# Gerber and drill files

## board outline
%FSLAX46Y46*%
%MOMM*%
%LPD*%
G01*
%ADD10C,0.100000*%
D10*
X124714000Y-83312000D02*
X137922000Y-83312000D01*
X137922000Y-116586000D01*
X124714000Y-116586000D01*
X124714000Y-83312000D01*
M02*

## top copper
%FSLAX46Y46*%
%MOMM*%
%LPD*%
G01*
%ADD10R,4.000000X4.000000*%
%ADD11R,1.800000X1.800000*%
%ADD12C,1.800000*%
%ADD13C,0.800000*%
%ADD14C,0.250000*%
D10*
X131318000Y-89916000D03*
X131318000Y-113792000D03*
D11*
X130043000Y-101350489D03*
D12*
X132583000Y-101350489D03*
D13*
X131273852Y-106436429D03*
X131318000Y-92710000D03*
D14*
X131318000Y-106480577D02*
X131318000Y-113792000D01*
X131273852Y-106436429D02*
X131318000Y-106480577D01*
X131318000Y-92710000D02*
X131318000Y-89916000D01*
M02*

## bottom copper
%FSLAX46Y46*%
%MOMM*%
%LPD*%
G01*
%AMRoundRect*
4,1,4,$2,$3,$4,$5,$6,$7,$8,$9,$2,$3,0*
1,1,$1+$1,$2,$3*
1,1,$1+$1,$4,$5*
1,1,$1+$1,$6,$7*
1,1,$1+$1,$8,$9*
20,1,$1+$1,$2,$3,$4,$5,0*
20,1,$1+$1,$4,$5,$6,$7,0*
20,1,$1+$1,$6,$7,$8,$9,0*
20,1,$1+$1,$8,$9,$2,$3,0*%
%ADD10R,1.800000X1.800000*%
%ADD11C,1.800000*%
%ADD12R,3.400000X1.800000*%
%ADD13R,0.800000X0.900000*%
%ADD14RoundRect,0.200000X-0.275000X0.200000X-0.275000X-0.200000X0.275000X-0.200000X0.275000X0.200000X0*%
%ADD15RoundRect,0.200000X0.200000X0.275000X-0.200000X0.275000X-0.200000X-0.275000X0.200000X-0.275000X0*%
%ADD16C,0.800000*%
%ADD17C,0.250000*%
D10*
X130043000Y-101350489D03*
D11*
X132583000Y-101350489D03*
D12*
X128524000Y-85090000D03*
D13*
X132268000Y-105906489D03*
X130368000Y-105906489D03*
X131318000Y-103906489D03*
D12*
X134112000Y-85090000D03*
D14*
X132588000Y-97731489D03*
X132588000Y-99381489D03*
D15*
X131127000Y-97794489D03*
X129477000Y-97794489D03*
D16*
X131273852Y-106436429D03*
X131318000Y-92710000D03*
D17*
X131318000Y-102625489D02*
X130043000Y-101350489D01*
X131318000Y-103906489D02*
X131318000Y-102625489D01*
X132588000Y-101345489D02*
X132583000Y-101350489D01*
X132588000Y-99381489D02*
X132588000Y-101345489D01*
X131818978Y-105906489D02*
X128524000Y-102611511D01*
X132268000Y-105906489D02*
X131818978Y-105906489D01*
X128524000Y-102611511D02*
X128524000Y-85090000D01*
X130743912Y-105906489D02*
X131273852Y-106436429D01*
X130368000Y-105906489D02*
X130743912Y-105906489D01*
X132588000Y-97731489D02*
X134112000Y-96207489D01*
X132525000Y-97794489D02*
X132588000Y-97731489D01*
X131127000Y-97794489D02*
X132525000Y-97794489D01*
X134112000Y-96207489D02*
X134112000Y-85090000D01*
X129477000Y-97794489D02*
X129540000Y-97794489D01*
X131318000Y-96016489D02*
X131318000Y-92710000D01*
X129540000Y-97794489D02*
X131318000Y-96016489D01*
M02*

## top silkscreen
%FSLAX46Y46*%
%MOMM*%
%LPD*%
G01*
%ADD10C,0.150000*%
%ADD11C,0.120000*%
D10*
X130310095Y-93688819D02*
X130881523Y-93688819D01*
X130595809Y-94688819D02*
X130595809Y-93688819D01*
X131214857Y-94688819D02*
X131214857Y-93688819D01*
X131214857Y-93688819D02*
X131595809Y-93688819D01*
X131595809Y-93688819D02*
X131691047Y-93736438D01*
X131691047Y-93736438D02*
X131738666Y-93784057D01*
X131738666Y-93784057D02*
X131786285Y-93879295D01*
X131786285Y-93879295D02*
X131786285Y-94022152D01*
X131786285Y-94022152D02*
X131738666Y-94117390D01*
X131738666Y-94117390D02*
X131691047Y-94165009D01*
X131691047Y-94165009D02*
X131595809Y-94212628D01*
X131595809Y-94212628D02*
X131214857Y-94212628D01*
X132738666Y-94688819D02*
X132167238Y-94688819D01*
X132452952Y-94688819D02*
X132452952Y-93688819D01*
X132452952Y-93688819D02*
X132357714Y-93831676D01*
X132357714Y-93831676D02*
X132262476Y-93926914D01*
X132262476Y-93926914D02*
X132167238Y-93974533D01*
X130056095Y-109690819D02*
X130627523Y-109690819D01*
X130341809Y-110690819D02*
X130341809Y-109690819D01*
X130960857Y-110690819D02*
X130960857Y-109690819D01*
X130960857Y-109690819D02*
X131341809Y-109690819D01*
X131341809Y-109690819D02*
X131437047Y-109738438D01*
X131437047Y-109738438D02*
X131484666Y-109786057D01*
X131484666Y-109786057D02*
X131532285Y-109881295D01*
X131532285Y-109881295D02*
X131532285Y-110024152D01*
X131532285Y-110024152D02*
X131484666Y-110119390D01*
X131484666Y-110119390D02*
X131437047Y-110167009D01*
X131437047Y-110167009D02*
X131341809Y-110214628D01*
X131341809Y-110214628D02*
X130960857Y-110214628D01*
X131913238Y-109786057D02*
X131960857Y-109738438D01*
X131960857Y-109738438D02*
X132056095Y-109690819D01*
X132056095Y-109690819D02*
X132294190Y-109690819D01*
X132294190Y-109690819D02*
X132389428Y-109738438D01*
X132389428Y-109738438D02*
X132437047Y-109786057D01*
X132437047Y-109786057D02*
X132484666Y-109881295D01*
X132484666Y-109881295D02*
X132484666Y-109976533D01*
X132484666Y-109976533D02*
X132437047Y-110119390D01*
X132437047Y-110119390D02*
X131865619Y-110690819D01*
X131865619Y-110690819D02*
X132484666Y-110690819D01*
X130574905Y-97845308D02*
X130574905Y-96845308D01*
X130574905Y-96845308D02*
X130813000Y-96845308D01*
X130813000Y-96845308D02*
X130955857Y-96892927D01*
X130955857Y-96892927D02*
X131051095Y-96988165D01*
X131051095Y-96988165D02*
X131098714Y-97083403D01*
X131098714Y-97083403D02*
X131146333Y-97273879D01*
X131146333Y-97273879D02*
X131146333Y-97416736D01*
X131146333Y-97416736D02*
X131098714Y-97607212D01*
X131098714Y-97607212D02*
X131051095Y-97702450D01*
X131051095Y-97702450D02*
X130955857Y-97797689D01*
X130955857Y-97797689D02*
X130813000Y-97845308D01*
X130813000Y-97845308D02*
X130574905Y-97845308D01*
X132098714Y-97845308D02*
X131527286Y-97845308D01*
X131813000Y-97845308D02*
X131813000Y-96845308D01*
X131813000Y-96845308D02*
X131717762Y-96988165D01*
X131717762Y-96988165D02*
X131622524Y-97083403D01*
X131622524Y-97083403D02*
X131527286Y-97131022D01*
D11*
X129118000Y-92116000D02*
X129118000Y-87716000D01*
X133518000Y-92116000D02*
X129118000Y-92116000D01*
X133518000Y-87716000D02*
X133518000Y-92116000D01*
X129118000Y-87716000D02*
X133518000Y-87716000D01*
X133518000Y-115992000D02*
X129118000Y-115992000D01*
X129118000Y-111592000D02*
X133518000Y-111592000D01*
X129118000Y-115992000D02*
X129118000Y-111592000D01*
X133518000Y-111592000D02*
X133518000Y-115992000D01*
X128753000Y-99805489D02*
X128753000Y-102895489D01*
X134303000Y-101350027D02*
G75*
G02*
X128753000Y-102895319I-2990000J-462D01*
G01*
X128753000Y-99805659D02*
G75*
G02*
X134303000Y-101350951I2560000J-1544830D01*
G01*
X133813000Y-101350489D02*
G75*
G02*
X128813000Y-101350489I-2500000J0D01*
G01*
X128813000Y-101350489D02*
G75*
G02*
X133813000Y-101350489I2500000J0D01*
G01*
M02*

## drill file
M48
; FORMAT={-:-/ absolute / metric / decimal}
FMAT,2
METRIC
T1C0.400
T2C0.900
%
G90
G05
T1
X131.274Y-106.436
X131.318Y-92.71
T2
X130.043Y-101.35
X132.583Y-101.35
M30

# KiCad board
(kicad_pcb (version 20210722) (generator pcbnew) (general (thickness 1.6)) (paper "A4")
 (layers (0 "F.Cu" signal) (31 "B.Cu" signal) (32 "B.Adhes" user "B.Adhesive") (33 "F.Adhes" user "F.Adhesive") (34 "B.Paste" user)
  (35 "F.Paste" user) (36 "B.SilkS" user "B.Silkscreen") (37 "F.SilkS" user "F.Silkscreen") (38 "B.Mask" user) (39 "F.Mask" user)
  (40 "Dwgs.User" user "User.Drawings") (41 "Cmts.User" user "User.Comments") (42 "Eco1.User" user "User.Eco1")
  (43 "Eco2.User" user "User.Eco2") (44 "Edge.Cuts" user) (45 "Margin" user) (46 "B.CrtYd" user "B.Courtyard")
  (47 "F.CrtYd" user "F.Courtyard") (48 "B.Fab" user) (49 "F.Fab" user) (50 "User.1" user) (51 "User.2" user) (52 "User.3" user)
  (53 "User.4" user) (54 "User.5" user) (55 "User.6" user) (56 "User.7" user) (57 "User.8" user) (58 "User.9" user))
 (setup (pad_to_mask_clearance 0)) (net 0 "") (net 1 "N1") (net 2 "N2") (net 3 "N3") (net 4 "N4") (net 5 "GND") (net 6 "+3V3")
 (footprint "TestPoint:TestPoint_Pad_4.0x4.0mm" (layer "F.Cu") (at 131.318 89.916)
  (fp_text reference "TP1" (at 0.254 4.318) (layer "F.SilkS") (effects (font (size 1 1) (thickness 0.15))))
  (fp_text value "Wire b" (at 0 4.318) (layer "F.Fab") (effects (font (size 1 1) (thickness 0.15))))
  (fp_line (start -2.2 2.2) (end -2.2 -2.2) (layer "F.SilkS") (width 0.12))
  (fp_line (start 2.2 2.2) (end -2.2 2.2) (layer "F.SilkS") (width 0.12))
  (fp_line (start 2.2 -2.2) (end 2.2 2.2) (layer "F.SilkS") (width 0.12))
  (fp_line (start -2.2 -2.2) (end 2.2 -2.2) (layer "F.SilkS") (width 0.12))
  (pad "1" smd rect locked (at 0 0) (size 4 4) (layers "F.Cu" "F.Mask") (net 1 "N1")))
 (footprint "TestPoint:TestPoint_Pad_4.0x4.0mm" (layer "F.Cu") (at 131.318 113.792)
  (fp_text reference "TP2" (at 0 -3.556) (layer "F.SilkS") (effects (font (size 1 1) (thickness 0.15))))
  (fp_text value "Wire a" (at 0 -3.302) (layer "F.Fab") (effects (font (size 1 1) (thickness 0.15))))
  (fp_line (start 2.2 2.2) (end -2.2 2.2) (layer "F.SilkS") (width 0.12))
  (fp_line (start -2.2 -2.2) (end 2.2 -2.2) (layer "F.SilkS") (width 0.12))
  (fp_line (start -2.2 2.2) (end -2.2 -2.2) (layer "F.SilkS") (width 0.12))
  (fp_line (start 2.2 -2.2) (end 2.2 2.2) (layer "F.SilkS") (width 0.12))
  (pad "1" smd rect locked (at 0 0) (size 4 4) (layers "F.Cu" "F.Mask") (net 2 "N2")))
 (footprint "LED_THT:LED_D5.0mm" (layer "F.Cu") (at 130.043 101.350489)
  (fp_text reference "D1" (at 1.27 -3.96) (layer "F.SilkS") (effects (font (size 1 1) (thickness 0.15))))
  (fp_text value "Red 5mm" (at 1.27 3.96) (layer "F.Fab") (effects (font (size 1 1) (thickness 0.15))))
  (fp_line (start -1.29 -1.545) (end -1.29 1.545) (layer "F.SilkS") (width 0.12))
  (fp_arc (start 1.27 0) (end -1.29 1.54483) (angle -148.9) (layer "F.SilkS") (width 0.12))
  (fp_arc (start 1.27 0) (end -1.29 -1.54483) (angle 148.9) (layer "F.SilkS") (width 0.12))
  (fp_circle (center 1.27 0) (end 3.77 0) (layer "F.SilkS") (width 0.12) (fill none))
  (pad "1" thru_hole rect locked (at 0 0) (size 1.8 1.8) (drill 0.9) (layers *.Cu *.Mask) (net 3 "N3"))
  (pad "2" thru_hole circle locked (at 2.54 0) (size 1.8 1.8) (drill 0.9) (layers *.Cu *.Mask) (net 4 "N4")))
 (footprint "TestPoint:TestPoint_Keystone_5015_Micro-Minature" (layer "B.Cu") (at 128.524 85.09)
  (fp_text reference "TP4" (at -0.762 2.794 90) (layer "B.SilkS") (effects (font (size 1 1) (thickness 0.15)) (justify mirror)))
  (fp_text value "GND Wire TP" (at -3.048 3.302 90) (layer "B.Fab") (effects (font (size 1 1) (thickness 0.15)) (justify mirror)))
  (pad "1" smd rect locked (at 0 0) (size 3.4 1.8) (layers "B.Cu" "B.Paste" "B.Mask") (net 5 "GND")))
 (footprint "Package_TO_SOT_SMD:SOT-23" (layer "B.Cu") (at 131.318 104.906489 90)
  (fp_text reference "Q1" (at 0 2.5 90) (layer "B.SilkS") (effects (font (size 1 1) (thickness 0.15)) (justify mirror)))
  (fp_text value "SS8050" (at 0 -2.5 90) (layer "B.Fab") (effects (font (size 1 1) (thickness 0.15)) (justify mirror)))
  (pad "1" smd rect locked (at -1 0.95 90) (size 0.9 0.8) (layers "B.Cu" "B.Paste" "B.Mask") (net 5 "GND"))
  (pad "2" smd rect locked (at -1 -0.95 90) (size 0.9 0.8) (layers "B.Cu" "B.Paste" "B.Mask") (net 2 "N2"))
  (pad "3" smd rect locked (at 1 0 90) (size 0.9 0.8) (layers "B.Cu" "B.Paste" "B.Mask") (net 3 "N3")))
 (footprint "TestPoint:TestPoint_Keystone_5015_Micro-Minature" (layer "B.Cu") (at 134.112 85.09)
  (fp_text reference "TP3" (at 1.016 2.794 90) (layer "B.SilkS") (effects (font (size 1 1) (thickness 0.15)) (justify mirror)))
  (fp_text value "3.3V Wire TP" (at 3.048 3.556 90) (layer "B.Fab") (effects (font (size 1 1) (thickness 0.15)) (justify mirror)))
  (pad "1" smd rect locked (at 0 0) (size 3.4 1.8) (layers "B.Cu" "B.Paste" "B.Mask") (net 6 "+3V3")))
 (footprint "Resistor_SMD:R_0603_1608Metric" (layer "B.Cu") (at 132.588 98.556489 -90)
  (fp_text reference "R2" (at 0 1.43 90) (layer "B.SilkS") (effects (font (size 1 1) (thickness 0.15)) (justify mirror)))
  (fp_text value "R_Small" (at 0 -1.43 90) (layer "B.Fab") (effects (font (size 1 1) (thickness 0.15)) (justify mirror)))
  (pad "1" smd roundrect locked (at -0.825 0 270) (size 0.8 0.95) (layers "B.Cu" "B.Paste" "B.Mask") (roundrect_rratio 0.25) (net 6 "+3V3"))
  (pad "2" smd roundrect locked (at 0.825 0 270) (size 0.8 0.95) (layers "B.Cu" "B.Paste" "B.Mask") (roundrect_rratio 0.25) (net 4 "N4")))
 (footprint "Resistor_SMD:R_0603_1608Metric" (layer "B.Cu") (at 130.302 97.794489 180)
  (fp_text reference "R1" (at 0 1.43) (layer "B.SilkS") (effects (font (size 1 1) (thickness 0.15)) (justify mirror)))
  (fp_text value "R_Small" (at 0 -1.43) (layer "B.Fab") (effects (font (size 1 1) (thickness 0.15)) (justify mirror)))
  (pad "1" smd roundrect locked (at -0.825 0 180) (size 0.8 0.95) (layers "B.Cu" "B.Paste" "B.Mask") (roundrect_rratio 0.25) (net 6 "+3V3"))
  (pad "2" smd roundrect locked (at 0.825 0 180) (size 0.8 0.95) (layers "B.Cu" "B.Paste" "B.Mask") (roundrect_rratio 0.25) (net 1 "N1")))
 (gr_rect (start 137.922 116.586) (end 124.714 83.312) (layer "Edge.Cuts") (width 0.1) (fill none))
 (segment (start 131.318 102.625489) (end 130.043 101.350489) (width 0.25) (layer "B.Cu") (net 3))
 (segment (start 131.318 103.906489) (end 131.318 102.625489) (width 0.25) (layer "B.Cu") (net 3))
 (segment (start 132.588 101.345489) (end 132.583 101.350489) (width 0.25) (layer "B.Cu") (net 4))
 (segment (start 132.588 99.381489) (end 132.588 101.345489) (width 0.25) (layer "B.Cu") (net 4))
 (segment (start 131.818978 105.906489) (end 128.524 102.611511) (width 0.25) (layer "B.Cu") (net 5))
 (segment (start 132.268 105.906489) (end 131.818978 105.906489) (width 0.25) (layer "B.Cu") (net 5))
 (segment (start 128.524 102.611511) (end 128.524 85.09) (width 0.25) (layer "B.Cu") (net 5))
 (segment (start 131.318 106.480577) (end 131.318 113.792) (width 0.25) (layer "F.Cu") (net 2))
 (segment (start 131.273852 106.436429) (end 131.318 106.480577) (width 0.25) (layer "F.Cu") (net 2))
 (via (at 131.273852 106.436429) (size 0.8) (drill 0.4) (layers "F.Cu" "B.Cu") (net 2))
 (segment (start 130.743912 105.906489) (end 131.273852 106.436429) (width 0.25) (layer "B.Cu") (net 2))
 (segment (start 130.368 105.906489) (end 130.743912 105.906489) (width 0.25) (layer "B.Cu") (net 2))
 (segment (start 132.588 97.731489) (end 134.112 96.207489) (width 0.25) (layer "B.Cu") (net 6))
 (segment (start 132.525 97.794489) (end 132.588 97.731489) (width 0.25) (layer "B.Cu") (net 6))
 (segment (start 131.127 97.794489) (end 132.525 97.794489) (width 0.25) (layer "B.Cu") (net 6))
 (segment (start 134.112 96.207489) (end 134.112 85.09) (width 0.25) (layer "B.Cu") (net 6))
 (segment (start 131.318 92.71) (end 131.318 89.916) (width 0.25) (layer "F.Cu") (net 1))
 (via (at 131.318 92.71) (size 0.8) (drill 0.4) (layers "F.Cu" "B.Cu") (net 1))
 (segment (start 129.477 97.794489) (end 129.54 97.794489) (width 0.25) (layer "B.Cu") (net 1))
 (segment (start 131.318 96.016489) (end 131.318 92.71) (width 0.25) (layer "B.Cu") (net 1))
 (segment (start 129.54 97.794489) (end 131.318 96.016489) (width 0.25) (layer "B.Cu") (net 1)))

